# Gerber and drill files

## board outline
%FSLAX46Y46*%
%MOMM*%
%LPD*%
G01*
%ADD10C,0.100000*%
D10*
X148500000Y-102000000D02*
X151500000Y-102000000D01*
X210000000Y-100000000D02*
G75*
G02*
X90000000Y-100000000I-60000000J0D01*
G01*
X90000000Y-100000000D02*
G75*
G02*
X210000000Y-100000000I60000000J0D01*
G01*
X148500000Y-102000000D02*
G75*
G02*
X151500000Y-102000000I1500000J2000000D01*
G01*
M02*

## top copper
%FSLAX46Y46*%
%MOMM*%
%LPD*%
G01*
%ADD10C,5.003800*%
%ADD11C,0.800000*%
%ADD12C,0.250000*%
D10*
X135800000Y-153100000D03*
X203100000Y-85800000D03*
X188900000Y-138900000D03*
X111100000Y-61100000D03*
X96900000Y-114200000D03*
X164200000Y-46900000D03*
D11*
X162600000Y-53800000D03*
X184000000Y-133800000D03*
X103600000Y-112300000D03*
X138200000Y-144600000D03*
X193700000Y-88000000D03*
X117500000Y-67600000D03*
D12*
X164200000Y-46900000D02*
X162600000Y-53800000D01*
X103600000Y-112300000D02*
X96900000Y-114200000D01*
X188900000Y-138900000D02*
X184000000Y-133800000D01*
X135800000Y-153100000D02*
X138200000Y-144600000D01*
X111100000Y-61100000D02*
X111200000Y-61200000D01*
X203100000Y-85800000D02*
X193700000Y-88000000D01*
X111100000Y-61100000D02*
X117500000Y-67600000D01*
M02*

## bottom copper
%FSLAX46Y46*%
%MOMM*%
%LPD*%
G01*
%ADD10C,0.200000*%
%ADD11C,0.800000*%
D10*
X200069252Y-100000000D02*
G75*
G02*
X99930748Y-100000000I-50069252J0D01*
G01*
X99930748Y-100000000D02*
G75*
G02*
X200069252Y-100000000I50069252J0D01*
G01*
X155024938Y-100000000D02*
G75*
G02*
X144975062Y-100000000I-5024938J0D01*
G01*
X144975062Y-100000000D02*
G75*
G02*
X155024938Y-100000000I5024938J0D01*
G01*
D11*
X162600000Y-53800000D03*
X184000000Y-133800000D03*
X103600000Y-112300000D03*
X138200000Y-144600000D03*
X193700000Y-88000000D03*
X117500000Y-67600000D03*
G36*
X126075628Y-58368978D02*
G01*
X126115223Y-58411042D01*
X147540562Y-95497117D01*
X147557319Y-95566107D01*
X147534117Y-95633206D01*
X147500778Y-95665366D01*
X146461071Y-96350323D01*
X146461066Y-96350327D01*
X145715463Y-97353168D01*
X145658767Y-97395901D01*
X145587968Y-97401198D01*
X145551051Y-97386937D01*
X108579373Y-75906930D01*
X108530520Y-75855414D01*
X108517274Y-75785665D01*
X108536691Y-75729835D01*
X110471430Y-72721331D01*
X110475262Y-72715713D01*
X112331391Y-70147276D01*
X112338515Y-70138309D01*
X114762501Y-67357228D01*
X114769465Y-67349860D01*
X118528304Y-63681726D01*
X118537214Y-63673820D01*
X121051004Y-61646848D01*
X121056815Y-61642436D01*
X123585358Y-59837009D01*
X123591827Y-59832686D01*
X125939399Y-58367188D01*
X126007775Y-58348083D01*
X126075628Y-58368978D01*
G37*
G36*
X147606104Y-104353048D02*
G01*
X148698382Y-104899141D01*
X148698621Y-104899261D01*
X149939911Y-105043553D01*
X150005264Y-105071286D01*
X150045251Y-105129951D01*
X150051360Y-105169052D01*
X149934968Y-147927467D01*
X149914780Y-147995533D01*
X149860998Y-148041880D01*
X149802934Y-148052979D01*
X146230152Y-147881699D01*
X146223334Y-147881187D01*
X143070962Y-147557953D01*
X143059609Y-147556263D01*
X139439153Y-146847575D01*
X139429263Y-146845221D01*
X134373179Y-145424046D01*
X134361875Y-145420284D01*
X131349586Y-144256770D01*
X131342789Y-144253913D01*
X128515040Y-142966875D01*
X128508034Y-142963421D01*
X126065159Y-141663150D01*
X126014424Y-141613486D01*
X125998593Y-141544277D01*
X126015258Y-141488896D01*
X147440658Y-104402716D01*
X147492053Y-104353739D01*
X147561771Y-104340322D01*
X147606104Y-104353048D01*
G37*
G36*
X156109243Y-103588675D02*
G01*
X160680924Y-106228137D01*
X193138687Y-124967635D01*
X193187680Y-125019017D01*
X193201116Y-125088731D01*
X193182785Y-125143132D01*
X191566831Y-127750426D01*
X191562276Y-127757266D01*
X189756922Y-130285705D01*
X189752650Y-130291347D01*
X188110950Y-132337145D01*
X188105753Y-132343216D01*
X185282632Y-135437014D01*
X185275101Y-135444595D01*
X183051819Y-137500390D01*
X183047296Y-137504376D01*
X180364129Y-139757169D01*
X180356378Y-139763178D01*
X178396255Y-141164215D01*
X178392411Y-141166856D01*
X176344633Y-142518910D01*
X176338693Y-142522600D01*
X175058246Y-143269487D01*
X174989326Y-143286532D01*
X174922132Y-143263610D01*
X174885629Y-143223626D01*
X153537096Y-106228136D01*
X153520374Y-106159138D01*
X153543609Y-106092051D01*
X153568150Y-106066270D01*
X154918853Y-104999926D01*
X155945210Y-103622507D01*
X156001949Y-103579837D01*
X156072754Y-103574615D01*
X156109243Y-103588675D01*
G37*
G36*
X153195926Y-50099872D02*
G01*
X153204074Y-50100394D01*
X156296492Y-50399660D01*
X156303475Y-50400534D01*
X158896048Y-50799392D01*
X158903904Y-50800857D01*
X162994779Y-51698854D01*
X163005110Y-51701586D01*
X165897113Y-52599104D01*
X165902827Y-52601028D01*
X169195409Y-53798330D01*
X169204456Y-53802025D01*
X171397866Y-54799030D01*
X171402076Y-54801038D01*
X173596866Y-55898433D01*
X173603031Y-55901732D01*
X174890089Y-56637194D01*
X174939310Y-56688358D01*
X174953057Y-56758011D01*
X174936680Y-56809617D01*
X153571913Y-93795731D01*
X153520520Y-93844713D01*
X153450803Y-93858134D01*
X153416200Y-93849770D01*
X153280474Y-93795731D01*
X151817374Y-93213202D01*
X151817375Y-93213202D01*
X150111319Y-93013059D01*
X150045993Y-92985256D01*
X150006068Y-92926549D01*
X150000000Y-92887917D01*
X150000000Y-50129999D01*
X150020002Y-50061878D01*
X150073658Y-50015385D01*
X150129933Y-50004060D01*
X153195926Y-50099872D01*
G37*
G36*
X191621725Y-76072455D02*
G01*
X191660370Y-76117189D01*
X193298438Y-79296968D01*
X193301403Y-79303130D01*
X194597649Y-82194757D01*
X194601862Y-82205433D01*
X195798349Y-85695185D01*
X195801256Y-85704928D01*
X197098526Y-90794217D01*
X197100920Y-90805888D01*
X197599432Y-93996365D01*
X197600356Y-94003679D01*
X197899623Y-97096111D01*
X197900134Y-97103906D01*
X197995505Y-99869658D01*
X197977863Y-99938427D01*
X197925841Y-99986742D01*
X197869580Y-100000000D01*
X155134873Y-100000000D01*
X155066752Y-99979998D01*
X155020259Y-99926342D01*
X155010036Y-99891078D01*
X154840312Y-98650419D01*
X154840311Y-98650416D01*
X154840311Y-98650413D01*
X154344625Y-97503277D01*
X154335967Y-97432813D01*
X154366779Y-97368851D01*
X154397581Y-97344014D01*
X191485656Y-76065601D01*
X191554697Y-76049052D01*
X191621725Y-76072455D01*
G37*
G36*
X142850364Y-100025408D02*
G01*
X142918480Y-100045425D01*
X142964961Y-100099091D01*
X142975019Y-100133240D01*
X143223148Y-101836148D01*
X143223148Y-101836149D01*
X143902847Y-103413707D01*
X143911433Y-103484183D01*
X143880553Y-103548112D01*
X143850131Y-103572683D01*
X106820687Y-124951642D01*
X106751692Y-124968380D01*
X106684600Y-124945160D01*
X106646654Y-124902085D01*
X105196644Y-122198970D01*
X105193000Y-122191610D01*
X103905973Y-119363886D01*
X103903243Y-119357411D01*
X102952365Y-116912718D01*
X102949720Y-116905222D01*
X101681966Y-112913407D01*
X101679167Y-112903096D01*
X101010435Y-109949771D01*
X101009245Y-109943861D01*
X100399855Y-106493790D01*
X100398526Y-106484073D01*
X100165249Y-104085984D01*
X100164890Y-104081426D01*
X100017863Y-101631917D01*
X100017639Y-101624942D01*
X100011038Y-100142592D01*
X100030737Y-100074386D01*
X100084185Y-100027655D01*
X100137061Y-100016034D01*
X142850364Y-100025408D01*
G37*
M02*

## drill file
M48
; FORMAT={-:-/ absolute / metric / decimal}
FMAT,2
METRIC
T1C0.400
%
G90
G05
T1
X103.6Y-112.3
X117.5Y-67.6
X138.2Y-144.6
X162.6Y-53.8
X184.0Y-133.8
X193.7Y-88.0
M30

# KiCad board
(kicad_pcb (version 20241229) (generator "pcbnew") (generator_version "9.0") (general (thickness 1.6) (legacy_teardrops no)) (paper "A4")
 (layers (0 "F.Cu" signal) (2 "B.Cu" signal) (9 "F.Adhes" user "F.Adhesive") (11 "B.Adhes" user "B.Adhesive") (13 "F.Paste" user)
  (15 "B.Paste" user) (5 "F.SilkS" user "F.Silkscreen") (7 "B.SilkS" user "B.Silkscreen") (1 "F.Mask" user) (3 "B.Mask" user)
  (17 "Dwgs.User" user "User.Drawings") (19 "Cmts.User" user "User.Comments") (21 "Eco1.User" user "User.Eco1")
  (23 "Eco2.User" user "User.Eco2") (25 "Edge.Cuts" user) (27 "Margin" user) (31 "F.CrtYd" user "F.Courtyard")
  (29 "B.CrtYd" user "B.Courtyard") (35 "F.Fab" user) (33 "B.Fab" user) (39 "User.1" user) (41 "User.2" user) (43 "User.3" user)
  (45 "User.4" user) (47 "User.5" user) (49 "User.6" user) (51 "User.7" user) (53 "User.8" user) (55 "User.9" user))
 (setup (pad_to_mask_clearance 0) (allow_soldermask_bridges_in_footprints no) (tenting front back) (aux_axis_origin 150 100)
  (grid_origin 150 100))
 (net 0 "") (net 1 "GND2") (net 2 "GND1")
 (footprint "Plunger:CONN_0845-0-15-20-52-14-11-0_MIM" (layer "F.Cu") (at 135.8 153.1 165)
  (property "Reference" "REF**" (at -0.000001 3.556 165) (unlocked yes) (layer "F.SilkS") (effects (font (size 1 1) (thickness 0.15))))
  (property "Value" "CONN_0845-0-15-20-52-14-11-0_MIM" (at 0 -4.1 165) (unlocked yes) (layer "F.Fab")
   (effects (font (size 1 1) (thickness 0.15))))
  (pad "1" smd circle (at 0 0 165) (size 5.0038 5.0038) (layers "F.Cu" "F.Mask" "F.Paste") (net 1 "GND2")))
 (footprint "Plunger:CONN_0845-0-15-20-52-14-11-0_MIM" (layer "F.Cu") (at 203.1 85.8 -75)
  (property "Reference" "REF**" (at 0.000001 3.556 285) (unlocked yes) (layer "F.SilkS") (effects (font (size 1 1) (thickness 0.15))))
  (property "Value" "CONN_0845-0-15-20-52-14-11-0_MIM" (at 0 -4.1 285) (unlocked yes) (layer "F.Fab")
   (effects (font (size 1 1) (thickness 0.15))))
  (pad "1" smd circle (at 0 0 285) (size 5.0038 5.0038) (layers "F.Cu" "F.Mask" "F.Paste") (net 1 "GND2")))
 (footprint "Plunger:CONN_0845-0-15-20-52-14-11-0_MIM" (layer "F.Cu") (at 188.9 138.9 -135)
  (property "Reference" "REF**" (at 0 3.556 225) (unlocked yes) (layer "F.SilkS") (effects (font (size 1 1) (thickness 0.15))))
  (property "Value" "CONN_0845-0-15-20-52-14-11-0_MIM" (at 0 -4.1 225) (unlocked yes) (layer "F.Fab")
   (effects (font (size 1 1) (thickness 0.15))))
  (pad "1" smd circle (at 0 0 225) (size 5.0038 5.0038) (layers "F.Cu" "F.Mask" "F.Paste") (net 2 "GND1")))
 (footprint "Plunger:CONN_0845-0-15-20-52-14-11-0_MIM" (layer "F.Cu") (at 111.1 61.1 45)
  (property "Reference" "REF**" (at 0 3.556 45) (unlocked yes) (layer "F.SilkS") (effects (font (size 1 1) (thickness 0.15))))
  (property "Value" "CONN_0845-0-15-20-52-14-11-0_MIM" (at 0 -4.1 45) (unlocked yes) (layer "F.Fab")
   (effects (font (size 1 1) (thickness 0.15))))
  (pad "1" smd circle (at 0 0 45) (size 5.0038 5.0038) (layers "F.Cu" "F.Mask" "F.Paste") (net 1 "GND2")))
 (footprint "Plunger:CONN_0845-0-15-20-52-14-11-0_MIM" (layer "F.Cu") (at 96.9 114.2 105)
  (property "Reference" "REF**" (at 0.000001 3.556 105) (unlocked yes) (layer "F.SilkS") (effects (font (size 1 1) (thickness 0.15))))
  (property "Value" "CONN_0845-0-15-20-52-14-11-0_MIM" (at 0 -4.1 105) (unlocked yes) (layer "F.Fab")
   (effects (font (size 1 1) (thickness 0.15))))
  (pad "1" smd circle (at 0 0 105) (size 5.0038 5.0038) (layers "F.Cu" "F.Mask" "F.Paste") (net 2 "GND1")))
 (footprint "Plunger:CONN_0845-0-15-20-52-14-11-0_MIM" (layer "F.Cu") (at 164.2 46.9 -16.9)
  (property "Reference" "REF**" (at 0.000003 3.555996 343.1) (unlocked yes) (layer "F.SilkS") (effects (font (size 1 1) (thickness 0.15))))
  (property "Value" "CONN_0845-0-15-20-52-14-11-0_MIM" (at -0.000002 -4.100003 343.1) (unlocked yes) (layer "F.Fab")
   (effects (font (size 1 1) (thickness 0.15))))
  (pad "1" smd circle (at 0 0 343.099) (size 5.0038 5.0038) (layers "F.Cu" "F.Mask" "F.Paste") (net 2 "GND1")))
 (gr_circle (center 150 100) (end 196.2 119.3) (stroke (width 0.2) (type solid)) (fill no) (layer "B.Cu") (net 2))
 (gr_circle (center 150 100) (end 153.4 103.7) (stroke (width 0.2) (type solid)) (fill no) (layer "B.Cu") (net 1))
 (gr_line (start 148.5 102) (end 151.5 102) (stroke (width 0.1) (type default)) (layer "Edge.Cuts"))
 (gr_circle (center 150 100) (end 210 100) (stroke (width 0.1) (type solid)) (fill no) (locked yes) (layer "Edge.Cuts"))
 (gr_arc (start 148.5 102) (mid 150 97.5) (end 151.5 102) (stroke (width 0.1) (type default)) (layer "Edge.Cuts"))
 (segment (start 164.2 46.9) (end 162.6 53.8) (width 0.25) (layer "F.Cu") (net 2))
 (segment (start 103.6 112.3) (end 96.9 114.2) (width 0.25) (layer "F.Cu") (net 2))
 (segment (start 188.9 138.9) (end 184 133.8) (width 0.25) (layer "F.Cu") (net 2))
 (via (at 162.6 53.8) (size 0.8) (drill 0.4) (layers "F.Cu" "B.Cu") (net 2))
 (via (at 184 133.8) (size 0.8) (drill 0.4) (layers "F.Cu" "B.Cu") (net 2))
 (via (at 103.6 112.3) (size 0.8) (drill 0.4) (layers "F.Cu" "B.Cu") (free yes) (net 2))
 (segment (start 135.8 153.1) (end 138.2 144.6) (width 0.25) (layer "F.Cu") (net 1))
 (segment (start 111.1 61.1) (end 111.2 61.2) (width 0.25) (layer "F.Cu") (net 1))
 (segment (start 203.1 85.8) (end 193.7 88) (width 0.25) (layer "F.Cu") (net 1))
 (segment (start 111.1 61.1) (end 117.5 67.6) (width 0.25) (layer "F.Cu") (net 1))
 (via (at 138.2 144.6) (size 0.8) (drill 0.4) (layers "F.Cu" "B.Cu") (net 1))
 (via (at 193.7 88) (size 0.8) (drill 0.4) (layers "F.Cu" "B.Cu") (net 1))
 (via (at 117.5 67.6) (size 0.8) (drill 0.4) (layers "F.Cu" "B.Cu") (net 1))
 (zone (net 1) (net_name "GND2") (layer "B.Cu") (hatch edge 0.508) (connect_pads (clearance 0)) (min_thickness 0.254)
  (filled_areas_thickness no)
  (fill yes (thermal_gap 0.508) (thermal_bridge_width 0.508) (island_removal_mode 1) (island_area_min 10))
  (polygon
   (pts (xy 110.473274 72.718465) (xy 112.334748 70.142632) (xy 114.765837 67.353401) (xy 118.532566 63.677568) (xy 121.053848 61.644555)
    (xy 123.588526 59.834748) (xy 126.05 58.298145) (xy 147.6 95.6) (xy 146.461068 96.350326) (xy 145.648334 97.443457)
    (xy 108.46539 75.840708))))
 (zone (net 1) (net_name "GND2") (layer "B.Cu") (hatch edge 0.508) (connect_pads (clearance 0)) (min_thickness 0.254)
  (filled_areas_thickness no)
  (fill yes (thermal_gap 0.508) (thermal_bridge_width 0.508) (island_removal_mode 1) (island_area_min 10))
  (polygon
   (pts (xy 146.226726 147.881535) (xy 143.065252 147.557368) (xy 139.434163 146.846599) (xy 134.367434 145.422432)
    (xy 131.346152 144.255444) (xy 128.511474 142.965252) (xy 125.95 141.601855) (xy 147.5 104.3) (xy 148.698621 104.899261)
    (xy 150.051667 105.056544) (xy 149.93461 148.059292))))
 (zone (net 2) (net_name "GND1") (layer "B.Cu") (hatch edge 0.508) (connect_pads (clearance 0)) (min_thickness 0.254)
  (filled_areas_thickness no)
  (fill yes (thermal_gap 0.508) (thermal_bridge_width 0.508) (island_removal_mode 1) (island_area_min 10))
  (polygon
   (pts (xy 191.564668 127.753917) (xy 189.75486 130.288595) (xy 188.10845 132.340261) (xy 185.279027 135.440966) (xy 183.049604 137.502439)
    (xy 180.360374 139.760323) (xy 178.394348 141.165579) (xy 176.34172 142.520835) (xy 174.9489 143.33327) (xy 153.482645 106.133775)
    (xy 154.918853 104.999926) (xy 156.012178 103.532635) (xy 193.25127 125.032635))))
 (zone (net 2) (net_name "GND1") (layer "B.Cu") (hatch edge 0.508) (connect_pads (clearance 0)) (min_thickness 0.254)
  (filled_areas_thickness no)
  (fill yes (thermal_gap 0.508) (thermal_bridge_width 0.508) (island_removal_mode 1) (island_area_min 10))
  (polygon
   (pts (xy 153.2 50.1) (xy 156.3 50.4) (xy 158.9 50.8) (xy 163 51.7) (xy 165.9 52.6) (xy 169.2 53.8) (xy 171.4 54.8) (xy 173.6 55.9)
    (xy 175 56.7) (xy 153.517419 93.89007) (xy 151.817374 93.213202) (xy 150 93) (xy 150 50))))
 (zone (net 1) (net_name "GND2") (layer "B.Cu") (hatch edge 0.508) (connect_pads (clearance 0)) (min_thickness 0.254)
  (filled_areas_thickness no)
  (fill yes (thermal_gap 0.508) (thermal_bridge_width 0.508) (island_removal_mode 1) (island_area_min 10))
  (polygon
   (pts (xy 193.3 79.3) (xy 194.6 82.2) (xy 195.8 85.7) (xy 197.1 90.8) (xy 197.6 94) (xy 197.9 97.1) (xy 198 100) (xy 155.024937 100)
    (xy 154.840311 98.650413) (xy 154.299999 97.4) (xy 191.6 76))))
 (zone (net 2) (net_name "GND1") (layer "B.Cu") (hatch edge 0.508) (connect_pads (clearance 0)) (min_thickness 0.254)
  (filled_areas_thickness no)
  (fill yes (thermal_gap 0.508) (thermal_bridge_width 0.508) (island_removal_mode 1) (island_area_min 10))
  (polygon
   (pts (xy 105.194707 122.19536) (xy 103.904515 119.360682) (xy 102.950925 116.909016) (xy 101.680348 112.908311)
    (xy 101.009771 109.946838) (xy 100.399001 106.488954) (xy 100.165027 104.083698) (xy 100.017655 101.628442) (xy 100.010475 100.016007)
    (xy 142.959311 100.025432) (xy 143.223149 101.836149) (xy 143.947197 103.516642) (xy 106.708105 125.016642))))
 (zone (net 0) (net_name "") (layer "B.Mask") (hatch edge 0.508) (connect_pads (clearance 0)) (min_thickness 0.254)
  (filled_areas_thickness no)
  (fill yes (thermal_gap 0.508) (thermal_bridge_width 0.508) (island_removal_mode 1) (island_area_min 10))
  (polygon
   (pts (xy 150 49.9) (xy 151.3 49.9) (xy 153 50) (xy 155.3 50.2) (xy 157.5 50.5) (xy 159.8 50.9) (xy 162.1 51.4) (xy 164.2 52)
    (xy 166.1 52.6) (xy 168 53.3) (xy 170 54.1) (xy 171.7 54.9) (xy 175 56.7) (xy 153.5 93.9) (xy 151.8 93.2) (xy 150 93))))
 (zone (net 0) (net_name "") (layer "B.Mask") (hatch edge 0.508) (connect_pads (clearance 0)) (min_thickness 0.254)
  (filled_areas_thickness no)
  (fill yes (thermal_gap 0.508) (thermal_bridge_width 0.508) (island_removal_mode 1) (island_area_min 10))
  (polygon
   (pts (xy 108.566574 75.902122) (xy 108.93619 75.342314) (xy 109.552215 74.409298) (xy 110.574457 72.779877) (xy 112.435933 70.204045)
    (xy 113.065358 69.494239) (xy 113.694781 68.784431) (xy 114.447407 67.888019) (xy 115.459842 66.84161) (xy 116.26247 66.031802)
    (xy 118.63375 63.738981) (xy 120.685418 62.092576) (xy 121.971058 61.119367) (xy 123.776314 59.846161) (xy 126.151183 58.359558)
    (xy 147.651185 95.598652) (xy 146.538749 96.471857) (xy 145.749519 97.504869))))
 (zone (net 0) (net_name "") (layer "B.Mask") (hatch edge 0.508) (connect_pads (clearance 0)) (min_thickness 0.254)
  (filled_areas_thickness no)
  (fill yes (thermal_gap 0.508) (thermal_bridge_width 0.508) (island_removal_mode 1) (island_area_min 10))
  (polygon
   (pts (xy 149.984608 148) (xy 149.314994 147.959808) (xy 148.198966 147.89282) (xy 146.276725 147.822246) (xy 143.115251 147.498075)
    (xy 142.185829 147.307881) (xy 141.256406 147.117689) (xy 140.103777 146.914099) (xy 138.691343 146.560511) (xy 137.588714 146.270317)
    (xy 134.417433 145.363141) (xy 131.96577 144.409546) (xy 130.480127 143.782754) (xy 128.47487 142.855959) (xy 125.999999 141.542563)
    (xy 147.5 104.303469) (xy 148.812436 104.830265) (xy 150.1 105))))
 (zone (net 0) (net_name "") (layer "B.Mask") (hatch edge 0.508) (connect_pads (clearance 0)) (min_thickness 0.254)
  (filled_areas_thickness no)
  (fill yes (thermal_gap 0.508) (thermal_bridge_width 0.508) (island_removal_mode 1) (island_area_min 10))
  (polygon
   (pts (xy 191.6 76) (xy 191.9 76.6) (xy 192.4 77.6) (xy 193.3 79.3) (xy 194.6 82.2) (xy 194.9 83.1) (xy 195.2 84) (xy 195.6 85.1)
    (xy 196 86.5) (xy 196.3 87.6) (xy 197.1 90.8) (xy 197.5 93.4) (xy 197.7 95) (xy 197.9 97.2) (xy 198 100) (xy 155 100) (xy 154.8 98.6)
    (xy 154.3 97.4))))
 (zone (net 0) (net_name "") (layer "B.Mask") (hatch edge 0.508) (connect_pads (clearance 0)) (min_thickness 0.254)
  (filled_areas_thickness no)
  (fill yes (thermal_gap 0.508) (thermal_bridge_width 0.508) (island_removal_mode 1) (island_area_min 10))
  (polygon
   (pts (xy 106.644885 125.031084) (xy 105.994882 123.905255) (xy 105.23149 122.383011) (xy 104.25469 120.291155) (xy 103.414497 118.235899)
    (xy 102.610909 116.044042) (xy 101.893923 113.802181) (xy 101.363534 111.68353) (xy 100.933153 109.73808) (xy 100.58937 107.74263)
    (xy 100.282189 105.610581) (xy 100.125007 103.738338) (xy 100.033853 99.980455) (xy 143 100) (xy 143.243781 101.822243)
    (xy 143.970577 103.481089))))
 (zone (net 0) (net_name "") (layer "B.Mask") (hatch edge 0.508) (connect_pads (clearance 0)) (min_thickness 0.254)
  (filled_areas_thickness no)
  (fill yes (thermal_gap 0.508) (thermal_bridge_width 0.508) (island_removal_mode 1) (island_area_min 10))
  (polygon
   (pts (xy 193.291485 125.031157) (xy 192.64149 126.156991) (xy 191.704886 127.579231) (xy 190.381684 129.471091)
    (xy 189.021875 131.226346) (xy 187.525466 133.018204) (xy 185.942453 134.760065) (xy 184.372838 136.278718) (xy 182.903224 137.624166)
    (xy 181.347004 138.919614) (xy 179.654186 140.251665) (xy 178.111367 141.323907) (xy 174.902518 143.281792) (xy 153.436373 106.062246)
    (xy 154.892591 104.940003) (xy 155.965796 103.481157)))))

